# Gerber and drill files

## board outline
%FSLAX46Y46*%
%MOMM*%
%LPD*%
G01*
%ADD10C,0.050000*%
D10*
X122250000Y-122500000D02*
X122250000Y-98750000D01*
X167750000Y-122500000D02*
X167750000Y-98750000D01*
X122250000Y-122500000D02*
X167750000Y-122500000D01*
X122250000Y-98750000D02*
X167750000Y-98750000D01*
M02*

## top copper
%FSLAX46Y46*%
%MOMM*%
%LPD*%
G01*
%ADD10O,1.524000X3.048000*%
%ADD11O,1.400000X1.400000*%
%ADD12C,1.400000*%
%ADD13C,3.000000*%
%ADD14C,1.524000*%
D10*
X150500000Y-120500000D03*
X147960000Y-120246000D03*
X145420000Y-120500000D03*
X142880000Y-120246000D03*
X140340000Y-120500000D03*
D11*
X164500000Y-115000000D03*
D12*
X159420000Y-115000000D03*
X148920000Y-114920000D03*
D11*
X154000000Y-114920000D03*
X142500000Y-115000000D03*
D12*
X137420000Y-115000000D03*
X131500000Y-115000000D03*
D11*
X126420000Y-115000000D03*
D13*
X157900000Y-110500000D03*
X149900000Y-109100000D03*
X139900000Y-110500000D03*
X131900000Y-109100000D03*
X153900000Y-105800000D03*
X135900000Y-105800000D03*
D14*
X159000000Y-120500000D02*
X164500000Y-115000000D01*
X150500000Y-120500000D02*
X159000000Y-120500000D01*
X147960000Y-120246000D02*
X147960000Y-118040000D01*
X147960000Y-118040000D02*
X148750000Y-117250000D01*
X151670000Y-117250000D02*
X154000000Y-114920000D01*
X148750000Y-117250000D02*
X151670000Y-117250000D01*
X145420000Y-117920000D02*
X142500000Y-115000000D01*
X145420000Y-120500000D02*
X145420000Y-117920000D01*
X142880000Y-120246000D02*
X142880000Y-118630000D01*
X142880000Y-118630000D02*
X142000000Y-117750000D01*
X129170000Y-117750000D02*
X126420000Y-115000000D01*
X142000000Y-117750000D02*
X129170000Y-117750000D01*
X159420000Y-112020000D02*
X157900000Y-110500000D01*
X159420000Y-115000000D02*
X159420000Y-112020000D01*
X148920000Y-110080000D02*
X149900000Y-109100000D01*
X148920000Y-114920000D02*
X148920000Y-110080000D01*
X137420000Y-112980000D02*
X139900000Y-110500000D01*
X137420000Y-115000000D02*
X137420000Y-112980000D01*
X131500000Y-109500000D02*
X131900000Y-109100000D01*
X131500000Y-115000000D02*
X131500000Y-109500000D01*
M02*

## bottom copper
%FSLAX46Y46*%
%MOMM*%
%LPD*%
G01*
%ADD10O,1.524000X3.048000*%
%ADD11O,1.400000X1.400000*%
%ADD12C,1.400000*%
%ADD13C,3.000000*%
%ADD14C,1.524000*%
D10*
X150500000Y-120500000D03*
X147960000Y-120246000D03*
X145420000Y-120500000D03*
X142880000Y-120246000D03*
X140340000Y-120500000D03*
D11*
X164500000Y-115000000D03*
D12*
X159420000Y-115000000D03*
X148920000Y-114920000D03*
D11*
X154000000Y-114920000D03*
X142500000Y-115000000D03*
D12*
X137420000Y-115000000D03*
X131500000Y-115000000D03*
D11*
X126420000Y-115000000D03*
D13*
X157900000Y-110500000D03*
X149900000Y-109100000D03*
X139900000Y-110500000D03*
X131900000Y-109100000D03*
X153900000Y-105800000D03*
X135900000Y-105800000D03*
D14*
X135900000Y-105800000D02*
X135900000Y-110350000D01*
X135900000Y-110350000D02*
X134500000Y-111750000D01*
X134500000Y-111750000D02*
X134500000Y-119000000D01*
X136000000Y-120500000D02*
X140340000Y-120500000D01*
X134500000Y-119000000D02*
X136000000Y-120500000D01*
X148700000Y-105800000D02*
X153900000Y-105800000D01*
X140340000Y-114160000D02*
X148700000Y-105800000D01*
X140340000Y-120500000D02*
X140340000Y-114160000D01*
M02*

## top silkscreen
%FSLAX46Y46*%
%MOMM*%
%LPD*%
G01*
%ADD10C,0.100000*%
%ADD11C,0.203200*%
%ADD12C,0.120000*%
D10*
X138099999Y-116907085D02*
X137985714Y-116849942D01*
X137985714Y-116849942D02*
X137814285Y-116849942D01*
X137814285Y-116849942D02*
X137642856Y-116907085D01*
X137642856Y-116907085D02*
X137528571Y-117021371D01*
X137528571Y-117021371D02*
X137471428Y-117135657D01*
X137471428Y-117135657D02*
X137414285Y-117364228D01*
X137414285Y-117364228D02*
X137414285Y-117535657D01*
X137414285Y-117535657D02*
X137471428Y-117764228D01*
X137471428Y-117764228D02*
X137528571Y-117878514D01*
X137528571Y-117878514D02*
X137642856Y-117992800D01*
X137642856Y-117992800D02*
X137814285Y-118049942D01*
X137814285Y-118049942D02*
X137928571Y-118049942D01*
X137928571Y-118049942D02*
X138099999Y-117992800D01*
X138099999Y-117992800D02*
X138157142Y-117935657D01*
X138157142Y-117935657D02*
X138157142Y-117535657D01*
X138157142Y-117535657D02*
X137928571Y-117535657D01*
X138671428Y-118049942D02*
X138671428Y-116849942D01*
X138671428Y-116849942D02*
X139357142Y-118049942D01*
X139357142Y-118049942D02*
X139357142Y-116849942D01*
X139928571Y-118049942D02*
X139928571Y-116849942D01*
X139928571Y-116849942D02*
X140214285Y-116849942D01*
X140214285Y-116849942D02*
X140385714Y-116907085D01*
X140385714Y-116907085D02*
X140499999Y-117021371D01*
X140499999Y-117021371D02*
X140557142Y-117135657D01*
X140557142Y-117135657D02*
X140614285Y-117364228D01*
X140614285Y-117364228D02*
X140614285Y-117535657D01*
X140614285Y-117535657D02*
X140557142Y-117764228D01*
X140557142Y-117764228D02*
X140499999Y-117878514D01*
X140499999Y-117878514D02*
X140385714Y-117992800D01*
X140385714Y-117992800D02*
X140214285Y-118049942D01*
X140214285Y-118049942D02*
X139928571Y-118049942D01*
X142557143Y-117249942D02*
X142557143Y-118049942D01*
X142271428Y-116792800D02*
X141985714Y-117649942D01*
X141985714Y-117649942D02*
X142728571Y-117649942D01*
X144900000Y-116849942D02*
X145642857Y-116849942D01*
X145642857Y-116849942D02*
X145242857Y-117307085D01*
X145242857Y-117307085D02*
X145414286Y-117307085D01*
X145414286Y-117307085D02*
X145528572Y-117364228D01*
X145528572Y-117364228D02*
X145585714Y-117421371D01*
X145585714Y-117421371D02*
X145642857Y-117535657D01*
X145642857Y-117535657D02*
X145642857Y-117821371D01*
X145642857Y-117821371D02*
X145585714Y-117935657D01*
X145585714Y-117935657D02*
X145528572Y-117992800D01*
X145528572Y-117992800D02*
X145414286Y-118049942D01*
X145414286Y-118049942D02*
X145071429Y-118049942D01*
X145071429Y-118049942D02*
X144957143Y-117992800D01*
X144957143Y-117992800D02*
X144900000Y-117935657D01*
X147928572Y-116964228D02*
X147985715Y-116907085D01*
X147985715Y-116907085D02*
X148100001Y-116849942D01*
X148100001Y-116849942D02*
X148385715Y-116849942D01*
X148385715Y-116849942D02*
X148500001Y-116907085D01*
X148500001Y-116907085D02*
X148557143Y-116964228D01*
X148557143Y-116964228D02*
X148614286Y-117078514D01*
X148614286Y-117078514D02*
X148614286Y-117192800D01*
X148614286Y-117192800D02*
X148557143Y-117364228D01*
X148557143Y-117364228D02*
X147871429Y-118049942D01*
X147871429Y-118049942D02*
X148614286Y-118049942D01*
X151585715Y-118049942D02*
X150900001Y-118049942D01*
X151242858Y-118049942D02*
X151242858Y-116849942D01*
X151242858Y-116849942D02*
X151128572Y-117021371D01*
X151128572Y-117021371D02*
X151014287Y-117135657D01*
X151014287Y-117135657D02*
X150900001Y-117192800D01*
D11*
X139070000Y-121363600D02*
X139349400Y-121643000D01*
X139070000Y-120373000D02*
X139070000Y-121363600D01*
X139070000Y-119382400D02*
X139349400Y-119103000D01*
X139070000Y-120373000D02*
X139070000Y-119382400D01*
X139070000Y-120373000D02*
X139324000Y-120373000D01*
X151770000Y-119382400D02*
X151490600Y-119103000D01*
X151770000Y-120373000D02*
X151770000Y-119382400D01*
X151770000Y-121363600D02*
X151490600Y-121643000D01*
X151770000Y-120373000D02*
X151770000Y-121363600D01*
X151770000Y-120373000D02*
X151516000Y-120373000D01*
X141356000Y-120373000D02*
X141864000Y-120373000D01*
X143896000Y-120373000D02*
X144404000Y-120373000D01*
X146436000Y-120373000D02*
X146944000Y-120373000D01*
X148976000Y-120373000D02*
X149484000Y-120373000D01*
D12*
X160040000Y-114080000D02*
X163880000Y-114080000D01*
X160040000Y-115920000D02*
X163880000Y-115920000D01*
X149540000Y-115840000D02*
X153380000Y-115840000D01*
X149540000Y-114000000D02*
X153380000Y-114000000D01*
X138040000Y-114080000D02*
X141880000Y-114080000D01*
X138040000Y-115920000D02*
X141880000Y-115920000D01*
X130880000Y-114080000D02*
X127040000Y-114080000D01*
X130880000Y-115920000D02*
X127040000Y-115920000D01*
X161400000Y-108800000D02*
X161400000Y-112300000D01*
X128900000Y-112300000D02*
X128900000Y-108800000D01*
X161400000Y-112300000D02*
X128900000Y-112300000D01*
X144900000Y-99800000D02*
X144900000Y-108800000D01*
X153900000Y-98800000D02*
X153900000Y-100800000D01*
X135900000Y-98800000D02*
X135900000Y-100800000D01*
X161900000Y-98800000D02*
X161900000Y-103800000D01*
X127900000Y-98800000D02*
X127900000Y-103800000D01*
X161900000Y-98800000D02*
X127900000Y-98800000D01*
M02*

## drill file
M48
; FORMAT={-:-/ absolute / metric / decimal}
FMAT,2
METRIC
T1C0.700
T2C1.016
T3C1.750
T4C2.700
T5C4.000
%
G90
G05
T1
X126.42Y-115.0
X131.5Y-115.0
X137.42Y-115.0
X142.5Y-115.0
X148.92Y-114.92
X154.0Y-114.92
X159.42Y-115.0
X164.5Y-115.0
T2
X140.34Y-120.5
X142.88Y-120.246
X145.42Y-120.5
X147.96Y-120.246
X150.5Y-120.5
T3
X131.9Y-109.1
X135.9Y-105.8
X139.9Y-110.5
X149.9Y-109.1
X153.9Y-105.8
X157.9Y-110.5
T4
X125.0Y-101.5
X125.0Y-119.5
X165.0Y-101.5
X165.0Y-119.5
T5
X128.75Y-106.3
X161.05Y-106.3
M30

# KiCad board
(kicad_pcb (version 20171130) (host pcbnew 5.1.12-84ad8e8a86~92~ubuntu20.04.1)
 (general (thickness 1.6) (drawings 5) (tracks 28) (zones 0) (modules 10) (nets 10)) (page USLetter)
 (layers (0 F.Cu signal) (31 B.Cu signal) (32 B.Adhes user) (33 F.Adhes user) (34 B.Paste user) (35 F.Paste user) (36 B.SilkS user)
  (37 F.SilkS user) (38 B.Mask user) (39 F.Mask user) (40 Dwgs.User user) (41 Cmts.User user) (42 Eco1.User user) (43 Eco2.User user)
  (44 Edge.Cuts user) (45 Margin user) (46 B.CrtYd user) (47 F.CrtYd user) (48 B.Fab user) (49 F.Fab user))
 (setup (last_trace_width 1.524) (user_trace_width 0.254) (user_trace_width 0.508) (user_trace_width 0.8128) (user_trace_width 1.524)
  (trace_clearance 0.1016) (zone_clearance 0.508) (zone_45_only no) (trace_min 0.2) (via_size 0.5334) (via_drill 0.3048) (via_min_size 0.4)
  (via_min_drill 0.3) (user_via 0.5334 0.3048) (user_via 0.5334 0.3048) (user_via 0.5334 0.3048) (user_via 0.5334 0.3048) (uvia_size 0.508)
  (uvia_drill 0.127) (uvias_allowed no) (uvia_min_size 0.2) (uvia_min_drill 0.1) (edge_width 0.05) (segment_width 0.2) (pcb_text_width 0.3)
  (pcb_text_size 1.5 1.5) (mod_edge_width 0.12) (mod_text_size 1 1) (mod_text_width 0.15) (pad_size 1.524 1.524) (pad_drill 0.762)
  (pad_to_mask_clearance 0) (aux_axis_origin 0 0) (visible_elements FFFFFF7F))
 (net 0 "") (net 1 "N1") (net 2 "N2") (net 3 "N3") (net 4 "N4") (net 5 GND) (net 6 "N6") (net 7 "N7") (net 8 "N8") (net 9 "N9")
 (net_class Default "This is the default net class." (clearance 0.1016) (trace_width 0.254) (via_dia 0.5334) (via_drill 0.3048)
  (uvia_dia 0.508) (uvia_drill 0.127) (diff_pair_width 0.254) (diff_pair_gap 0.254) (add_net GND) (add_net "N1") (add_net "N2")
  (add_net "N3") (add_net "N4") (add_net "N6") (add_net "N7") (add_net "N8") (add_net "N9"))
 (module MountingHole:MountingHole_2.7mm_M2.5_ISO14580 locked (layer F.Cu) (at 165 101.5)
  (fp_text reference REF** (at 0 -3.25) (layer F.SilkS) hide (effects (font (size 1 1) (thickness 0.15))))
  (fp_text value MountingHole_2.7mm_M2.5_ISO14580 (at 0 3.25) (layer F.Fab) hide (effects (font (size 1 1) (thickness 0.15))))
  (pad 1 np_thru_hole circle (at 0 0) (size 2.7 2.7) (drill 2.7) (layers *.Cu *.Mask)))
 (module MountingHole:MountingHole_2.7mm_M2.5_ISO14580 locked (layer F.Cu) (at 125 119.5)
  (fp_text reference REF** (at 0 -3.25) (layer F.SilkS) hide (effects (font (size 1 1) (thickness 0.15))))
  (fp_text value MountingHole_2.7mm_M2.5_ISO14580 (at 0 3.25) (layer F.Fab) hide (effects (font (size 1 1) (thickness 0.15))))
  (pad 1 np_thru_hole circle (at 0 0) (size 2.7 2.7) (drill 2.7) (layers *.Cu *.Mask)))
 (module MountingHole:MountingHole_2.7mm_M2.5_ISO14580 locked (layer F.Cu) (at 165 119.5)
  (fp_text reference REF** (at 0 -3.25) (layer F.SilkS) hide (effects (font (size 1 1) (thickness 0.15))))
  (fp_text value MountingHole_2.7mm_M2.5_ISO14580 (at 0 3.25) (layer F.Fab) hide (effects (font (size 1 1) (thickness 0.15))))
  (pad 1 np_thru_hole circle (at 0 0) (size 2.7 2.7) (drill 2.7) (layers *.Cu *.Mask)))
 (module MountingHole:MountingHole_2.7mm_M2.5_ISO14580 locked (layer F.Cu) (at 125 101.5)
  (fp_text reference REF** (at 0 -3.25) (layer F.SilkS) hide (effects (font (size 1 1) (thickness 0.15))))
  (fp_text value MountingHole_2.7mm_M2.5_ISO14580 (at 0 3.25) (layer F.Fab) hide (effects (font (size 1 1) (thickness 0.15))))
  (pad 1 np_thru_hole circle (at 0 0) (size 2.7 2.7) (drill 2.7) (layers *.Cu *.Mask)))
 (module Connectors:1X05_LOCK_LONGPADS (layer F.Cu) (at 150.5 120.5 180)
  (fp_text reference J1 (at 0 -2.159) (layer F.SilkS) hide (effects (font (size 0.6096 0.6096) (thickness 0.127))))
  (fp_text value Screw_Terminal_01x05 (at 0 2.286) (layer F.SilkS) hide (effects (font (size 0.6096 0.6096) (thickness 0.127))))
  (fp_line (start 11.43 -0.8636) (end 11.1506 -1.143) (layer F.SilkS) (width 0.2032))
  (fp_line (start 11.43 0.127) (end 11.43 -0.8636) (layer F.SilkS) (width 0.2032))
  (fp_line (start 11.43 1.1176) (end 11.1506 1.397) (layer F.SilkS) (width 0.2032))
  (fp_line (start 11.43 0.127) (end 11.43 1.1176) (layer F.SilkS) (width 0.2032))
  (fp_line (start 11.43 0.127) (end 11.176 0.127) (layer F.SilkS) (width 0.2032))
  (fp_line (start -1.27 1.1176) (end -0.9906 1.397) (layer F.SilkS) (width 0.2032))
  (fp_line (start -1.27 0.127) (end -1.27 1.1176) (layer F.SilkS) (width 0.2032))
  (fp_line (start -1.27 -0.8636) (end -0.9906 -1.143) (layer F.SilkS) (width 0.2032))
  (fp_line (start -1.27 0.127) (end -1.27 -0.8636) (layer F.SilkS) (width 0.2032))
  (fp_line (start -1.27 0.127) (end -1.016 0.127) (layer F.SilkS) (width 0.2032))
  (fp_line (start 9.144 0.127) (end 8.636 0.127) (layer F.SilkS) (width 0.2032))
  (fp_line (start 6.604 0.127) (end 6.096 0.127) (layer F.SilkS) (width 0.2032))
  (fp_line (start 4.064 0.127) (end 3.556 0.127) (layer F.SilkS) (width 0.2032))
  (fp_line (start 1.524 0.127) (end 1.016 0.127) (layer F.SilkS) (width 0.2032))
  (pad 1 thru_hole oval (at 0 0) (size 1.524 3.048) (drill 1.016) (layers *.Cu *.Mask) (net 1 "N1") (solder_mask_margin 0.1016))
  (pad 2 thru_hole oval (at 2.54 0.254) (size 1.524 3.048) (drill 1.016) (layers *.Cu *.Mask) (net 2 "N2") (solder_mask_margin 0.1016))
  (pad 3 thru_hole oval (at 5.08 0) (size 1.524 3.048) (drill 1.016) (layers *.Cu *.Mask) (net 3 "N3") (solder_mask_margin 0.1016))
  (pad 4 thru_hole oval (at 7.62 0.254) (size 1.524 3.048) (drill 1.016) (layers *.Cu *.Mask) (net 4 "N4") (solder_mask_margin 0.1016))
  (pad 5 thru_hole oval (at 10.16 0) (size 1.524 3.048) (drill 1.016) (layers *.Cu *.Mask) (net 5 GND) (solder_mask_margin 0.1016)))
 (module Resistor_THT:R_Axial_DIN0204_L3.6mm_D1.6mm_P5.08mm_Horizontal (layer F.Cu) (at 159.42 115)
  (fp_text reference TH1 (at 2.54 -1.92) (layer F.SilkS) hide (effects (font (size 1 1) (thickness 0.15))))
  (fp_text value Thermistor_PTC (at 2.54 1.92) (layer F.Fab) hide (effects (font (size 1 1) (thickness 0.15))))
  (fp_line (start 0.62 -0.92) (end 4.46 -0.92) (layer F.SilkS) (width 0.12))
  (fp_line (start 0.62 0.92) (end 4.46 0.92) (layer F.SilkS) (width 0.12))
  (pad 2 thru_hole oval (at 5.08 0) (size 1.4 1.4) (drill 0.7) (layers *.Cu *.Mask) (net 1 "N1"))
  (pad 1 thru_hole circle (at 0 0) (size 1.4 1.4) (drill 0.7) (layers *.Cu *.Mask) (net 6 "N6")))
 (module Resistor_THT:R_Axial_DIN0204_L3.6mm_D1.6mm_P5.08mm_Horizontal (layer F.Cu) (at 148.92 114.92)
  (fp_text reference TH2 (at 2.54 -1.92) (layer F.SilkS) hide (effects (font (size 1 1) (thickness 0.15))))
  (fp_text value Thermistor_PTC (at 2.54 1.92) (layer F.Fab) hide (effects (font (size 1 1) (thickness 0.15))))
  (fp_line (start 0.62 0.92) (end 4.46 0.92) (layer F.SilkS) (width 0.12))
  (fp_line (start 0.62 -0.92) (end 4.46 -0.92) (layer F.SilkS) (width 0.12))
  (pad 1 thru_hole circle (at 0 0) (size 1.4 1.4) (drill 0.7) (layers *.Cu *.Mask) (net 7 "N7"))
  (pad 2 thru_hole oval (at 5.08 0) (size 1.4 1.4) (drill 0.7) (layers *.Cu *.Mask) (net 2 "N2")))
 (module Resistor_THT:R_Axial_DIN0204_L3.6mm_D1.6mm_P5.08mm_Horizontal (layer F.Cu) (at 137.42 115)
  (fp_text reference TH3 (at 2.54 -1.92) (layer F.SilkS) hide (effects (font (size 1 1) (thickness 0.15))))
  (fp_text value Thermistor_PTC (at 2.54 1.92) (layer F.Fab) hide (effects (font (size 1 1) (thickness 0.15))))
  (fp_line (start 0.62 -0.92) (end 4.46 -0.92) (layer F.SilkS) (width 0.12))
  (fp_line (start 0.62 0.92) (end 4.46 0.92) (layer F.SilkS) (width 0.12))
  (pad 2 thru_hole oval (at 5.08 0) (size 1.4 1.4) (drill 0.7) (layers *.Cu *.Mask) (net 3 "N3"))
  (pad 1 thru_hole circle (at 0 0) (size 1.4 1.4) (drill 0.7) (layers *.Cu *.Mask) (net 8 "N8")))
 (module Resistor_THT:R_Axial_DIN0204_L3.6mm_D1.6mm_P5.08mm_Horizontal (layer F.Cu) (at 131.5 115 180)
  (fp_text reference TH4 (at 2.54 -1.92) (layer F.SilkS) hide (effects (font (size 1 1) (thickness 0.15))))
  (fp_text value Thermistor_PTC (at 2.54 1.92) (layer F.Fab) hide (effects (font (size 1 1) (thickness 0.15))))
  (fp_line (start 0.62 0.92) (end 4.46 0.92) (layer F.SilkS) (width 0.12))
  (fp_line (start 0.62 -0.92) (end 4.46 -0.92) (layer F.SilkS) (width 0.12))
  (pad 1 thru_hole circle (at 0 0 180) (size 1.4 1.4) (drill 0.7) (layers *.Cu *.Mask) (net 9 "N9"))
  (pad 2 thru_hole oval (at 5.08 0 180) (size 1.4 1.4) (drill 0.7) (layers *.Cu *.Mask) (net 4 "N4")))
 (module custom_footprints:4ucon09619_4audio (layer F.Cu) (at 144.9 105.8 180)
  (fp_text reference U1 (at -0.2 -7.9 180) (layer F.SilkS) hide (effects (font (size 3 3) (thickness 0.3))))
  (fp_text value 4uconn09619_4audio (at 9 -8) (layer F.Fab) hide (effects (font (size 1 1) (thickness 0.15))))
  (fp_line (start -16.5 -3) (end -16.5 -6.5) (layer F.SilkS) (width 0.12))
  (fp_line (start 16 -6.5) (end 16 -3) (layer F.SilkS) (width 0.12))
  (fp_line (start -16.5 -6.5) (end 16 -6.5) (layer F.SilkS) (width 0.12))
  (fp_line (start 0 6) (end 0 -3) (layer F.SilkS) (width 0.12))
  (fp_line (start -9 7) (end -9 5) (layer F.SilkS) (width 0.12)) (fp_line (start 9 7) (end 9 5) (layer F.SilkS) (width 0.12))
  (fp_line (start -17 7) (end -17 2) (layer F.SilkS) (width 0.12))
  (fp_line (start 17 7) (end 17 2) (layer F.SilkS) (width 0.12))
  (fp_line (start -17 7) (end 17 7) (layer F.SilkS) (width 0.12))
  (pad 1 thru_hole circle (at -13 -4.7 180) (size 3 3) (drill 1.75) (layers *.Cu *.Mask) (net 6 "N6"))
  (pad 2 thru_hole circle (at -5 -3.3 180) (size 3 3) (drill 1.75) (layers *.Cu *.Mask) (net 7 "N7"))
  (pad 3 thru_hole circle (at 5 -4.7 180) (size 3 3) (drill 1.75) (layers *.Cu *.Mask) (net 8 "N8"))
  (pad 4 thru_hole circle (at 13 -3.3 180) (size 3 3) (drill 1.75) (layers *.Cu *.Mask) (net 9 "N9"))
  (pad 5 thru_hole circle (at -9 0 180) (size 3 3) (drill 1.75) (layers *.Cu *.Mask) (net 5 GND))
  (pad 6 thru_hole circle (at 9 0 180) (size 3 3) (drill 1.75) (layers *.Cu *.Mask) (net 5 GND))
  (pad "" np_thru_hole circle (at -16.15 -0.5 180) (size 4 4) (drill 4) (layers *.Cu *.Mask))
  (pad "" np_thru_hole circle (at 16.15 -0.5 180) (size 4 4) (drill 4) (layers *.Cu *.Mask)))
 (gr_line (start 122.25 122.5) (end 122.25 98.75) (layer Edge.Cuts) (width 0.05))
 (gr_line (start 167.75 122.5) (end 167.75 98.75) (layer Edge.Cuts) (width 0.05))
 (gr_line (start 122.25 122.5) (end 167.75 122.5) (layer Edge.Cuts) (width 0.05))
 (gr_line (start 122.25 98.75) (end 167.75 98.75) (layer Edge.Cuts) (width 0.05))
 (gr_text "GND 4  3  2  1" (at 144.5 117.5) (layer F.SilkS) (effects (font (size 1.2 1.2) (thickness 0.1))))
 (segment (start 159 120.5) (end 164.5 115) (width 1.524) (layer F.Cu) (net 1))
 (segment (start 150.5 120.5) (end 159 120.5) (width 1.524) (layer F.Cu) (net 1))
 (segment (start 147.96 120.246) (end 147.96 118.04) (width 1.524) (layer F.Cu) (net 2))
 (segment (start 147.96 118.04) (end 148.75 117.25) (width 1.524) (layer F.Cu) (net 2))
 (segment (start 151.67 117.25) (end 154 114.92) (width 1.524) (layer F.Cu) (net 2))
 (segment (start 148.75 117.25) (end 151.67 117.25) (width 1.524) (layer F.Cu) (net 2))
 (segment (start 145.42 117.92) (end 142.5 115) (width 1.524) (layer F.Cu) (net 3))
 (segment (start 145.42 120.5) (end 145.42 117.92) (width 1.524) (layer F.Cu) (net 3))
 (segment (start 142.88 120.246) (end 142.88 118.63) (width 1.524) (layer F.Cu) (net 4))
 (segment (start 142.88 118.63) (end 142 117.75) (width 1.524) (layer F.Cu) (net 4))
 (segment (start 129.17 117.75) (end 126.42 115) (width 1.524) (layer F.Cu) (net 4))
 (segment (start 142 117.75) (end 129.17 117.75) (width 1.524) (layer F.Cu) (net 4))
 (segment (start 135.9 105.8) (end 135.9 110.35) (width 1.524) (layer B.Cu) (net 5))
 (segment (start 135.9 110.35) (end 134.5 111.75) (width 1.524) (layer B.Cu) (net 5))
 (segment (start 134.5 111.75) (end 134.5 119) (width 1.524) (layer B.Cu) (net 5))
 (segment (start 136 120.5) (end 140.34 120.5) (width 1.524) (layer B.Cu) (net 5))
 (segment (start 134.5 119) (end 136 120.5) (width 1.524) (layer B.Cu) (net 5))
 (segment (start 148.7 105.8) (end 153.9 105.8) (width 1.524) (layer B.Cu) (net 5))
 (segment (start 140.34 114.16) (end 148.7 105.8) (width 1.524) (layer B.Cu) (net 5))
 (segment (start 140.34 120.5) (end 140.34 114.16) (width 1.524) (layer B.Cu) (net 5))
 (segment (start 159.42 112.02) (end 157.9 110.5) (width 1.524) (layer F.Cu) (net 6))
 (segment (start 159.42 115) (end 159.42 112.02) (width 1.524) (layer F.Cu) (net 6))
 (segment (start 148.92 110.08) (end 149.9 109.1) (width 1.524) (layer F.Cu) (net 7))
 (segment (start 148.92 114.92) (end 148.92 110.08) (width 1.524) (layer F.Cu) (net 7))
 (segment (start 137.42 112.98) (end 139.9 110.5) (width 1.524) (layer F.Cu) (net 8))
 (segment (start 137.42 115) (end 137.42 112.98) (width 1.524) (layer F.Cu) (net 8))
 (segment (start 131.5 109.5) (end 131.9 109.1) (width 1.524) (layer F.Cu) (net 9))
 (segment (start 131.5 115) (end 131.5 109.5) (width 1.524) (layer F.Cu) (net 9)))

